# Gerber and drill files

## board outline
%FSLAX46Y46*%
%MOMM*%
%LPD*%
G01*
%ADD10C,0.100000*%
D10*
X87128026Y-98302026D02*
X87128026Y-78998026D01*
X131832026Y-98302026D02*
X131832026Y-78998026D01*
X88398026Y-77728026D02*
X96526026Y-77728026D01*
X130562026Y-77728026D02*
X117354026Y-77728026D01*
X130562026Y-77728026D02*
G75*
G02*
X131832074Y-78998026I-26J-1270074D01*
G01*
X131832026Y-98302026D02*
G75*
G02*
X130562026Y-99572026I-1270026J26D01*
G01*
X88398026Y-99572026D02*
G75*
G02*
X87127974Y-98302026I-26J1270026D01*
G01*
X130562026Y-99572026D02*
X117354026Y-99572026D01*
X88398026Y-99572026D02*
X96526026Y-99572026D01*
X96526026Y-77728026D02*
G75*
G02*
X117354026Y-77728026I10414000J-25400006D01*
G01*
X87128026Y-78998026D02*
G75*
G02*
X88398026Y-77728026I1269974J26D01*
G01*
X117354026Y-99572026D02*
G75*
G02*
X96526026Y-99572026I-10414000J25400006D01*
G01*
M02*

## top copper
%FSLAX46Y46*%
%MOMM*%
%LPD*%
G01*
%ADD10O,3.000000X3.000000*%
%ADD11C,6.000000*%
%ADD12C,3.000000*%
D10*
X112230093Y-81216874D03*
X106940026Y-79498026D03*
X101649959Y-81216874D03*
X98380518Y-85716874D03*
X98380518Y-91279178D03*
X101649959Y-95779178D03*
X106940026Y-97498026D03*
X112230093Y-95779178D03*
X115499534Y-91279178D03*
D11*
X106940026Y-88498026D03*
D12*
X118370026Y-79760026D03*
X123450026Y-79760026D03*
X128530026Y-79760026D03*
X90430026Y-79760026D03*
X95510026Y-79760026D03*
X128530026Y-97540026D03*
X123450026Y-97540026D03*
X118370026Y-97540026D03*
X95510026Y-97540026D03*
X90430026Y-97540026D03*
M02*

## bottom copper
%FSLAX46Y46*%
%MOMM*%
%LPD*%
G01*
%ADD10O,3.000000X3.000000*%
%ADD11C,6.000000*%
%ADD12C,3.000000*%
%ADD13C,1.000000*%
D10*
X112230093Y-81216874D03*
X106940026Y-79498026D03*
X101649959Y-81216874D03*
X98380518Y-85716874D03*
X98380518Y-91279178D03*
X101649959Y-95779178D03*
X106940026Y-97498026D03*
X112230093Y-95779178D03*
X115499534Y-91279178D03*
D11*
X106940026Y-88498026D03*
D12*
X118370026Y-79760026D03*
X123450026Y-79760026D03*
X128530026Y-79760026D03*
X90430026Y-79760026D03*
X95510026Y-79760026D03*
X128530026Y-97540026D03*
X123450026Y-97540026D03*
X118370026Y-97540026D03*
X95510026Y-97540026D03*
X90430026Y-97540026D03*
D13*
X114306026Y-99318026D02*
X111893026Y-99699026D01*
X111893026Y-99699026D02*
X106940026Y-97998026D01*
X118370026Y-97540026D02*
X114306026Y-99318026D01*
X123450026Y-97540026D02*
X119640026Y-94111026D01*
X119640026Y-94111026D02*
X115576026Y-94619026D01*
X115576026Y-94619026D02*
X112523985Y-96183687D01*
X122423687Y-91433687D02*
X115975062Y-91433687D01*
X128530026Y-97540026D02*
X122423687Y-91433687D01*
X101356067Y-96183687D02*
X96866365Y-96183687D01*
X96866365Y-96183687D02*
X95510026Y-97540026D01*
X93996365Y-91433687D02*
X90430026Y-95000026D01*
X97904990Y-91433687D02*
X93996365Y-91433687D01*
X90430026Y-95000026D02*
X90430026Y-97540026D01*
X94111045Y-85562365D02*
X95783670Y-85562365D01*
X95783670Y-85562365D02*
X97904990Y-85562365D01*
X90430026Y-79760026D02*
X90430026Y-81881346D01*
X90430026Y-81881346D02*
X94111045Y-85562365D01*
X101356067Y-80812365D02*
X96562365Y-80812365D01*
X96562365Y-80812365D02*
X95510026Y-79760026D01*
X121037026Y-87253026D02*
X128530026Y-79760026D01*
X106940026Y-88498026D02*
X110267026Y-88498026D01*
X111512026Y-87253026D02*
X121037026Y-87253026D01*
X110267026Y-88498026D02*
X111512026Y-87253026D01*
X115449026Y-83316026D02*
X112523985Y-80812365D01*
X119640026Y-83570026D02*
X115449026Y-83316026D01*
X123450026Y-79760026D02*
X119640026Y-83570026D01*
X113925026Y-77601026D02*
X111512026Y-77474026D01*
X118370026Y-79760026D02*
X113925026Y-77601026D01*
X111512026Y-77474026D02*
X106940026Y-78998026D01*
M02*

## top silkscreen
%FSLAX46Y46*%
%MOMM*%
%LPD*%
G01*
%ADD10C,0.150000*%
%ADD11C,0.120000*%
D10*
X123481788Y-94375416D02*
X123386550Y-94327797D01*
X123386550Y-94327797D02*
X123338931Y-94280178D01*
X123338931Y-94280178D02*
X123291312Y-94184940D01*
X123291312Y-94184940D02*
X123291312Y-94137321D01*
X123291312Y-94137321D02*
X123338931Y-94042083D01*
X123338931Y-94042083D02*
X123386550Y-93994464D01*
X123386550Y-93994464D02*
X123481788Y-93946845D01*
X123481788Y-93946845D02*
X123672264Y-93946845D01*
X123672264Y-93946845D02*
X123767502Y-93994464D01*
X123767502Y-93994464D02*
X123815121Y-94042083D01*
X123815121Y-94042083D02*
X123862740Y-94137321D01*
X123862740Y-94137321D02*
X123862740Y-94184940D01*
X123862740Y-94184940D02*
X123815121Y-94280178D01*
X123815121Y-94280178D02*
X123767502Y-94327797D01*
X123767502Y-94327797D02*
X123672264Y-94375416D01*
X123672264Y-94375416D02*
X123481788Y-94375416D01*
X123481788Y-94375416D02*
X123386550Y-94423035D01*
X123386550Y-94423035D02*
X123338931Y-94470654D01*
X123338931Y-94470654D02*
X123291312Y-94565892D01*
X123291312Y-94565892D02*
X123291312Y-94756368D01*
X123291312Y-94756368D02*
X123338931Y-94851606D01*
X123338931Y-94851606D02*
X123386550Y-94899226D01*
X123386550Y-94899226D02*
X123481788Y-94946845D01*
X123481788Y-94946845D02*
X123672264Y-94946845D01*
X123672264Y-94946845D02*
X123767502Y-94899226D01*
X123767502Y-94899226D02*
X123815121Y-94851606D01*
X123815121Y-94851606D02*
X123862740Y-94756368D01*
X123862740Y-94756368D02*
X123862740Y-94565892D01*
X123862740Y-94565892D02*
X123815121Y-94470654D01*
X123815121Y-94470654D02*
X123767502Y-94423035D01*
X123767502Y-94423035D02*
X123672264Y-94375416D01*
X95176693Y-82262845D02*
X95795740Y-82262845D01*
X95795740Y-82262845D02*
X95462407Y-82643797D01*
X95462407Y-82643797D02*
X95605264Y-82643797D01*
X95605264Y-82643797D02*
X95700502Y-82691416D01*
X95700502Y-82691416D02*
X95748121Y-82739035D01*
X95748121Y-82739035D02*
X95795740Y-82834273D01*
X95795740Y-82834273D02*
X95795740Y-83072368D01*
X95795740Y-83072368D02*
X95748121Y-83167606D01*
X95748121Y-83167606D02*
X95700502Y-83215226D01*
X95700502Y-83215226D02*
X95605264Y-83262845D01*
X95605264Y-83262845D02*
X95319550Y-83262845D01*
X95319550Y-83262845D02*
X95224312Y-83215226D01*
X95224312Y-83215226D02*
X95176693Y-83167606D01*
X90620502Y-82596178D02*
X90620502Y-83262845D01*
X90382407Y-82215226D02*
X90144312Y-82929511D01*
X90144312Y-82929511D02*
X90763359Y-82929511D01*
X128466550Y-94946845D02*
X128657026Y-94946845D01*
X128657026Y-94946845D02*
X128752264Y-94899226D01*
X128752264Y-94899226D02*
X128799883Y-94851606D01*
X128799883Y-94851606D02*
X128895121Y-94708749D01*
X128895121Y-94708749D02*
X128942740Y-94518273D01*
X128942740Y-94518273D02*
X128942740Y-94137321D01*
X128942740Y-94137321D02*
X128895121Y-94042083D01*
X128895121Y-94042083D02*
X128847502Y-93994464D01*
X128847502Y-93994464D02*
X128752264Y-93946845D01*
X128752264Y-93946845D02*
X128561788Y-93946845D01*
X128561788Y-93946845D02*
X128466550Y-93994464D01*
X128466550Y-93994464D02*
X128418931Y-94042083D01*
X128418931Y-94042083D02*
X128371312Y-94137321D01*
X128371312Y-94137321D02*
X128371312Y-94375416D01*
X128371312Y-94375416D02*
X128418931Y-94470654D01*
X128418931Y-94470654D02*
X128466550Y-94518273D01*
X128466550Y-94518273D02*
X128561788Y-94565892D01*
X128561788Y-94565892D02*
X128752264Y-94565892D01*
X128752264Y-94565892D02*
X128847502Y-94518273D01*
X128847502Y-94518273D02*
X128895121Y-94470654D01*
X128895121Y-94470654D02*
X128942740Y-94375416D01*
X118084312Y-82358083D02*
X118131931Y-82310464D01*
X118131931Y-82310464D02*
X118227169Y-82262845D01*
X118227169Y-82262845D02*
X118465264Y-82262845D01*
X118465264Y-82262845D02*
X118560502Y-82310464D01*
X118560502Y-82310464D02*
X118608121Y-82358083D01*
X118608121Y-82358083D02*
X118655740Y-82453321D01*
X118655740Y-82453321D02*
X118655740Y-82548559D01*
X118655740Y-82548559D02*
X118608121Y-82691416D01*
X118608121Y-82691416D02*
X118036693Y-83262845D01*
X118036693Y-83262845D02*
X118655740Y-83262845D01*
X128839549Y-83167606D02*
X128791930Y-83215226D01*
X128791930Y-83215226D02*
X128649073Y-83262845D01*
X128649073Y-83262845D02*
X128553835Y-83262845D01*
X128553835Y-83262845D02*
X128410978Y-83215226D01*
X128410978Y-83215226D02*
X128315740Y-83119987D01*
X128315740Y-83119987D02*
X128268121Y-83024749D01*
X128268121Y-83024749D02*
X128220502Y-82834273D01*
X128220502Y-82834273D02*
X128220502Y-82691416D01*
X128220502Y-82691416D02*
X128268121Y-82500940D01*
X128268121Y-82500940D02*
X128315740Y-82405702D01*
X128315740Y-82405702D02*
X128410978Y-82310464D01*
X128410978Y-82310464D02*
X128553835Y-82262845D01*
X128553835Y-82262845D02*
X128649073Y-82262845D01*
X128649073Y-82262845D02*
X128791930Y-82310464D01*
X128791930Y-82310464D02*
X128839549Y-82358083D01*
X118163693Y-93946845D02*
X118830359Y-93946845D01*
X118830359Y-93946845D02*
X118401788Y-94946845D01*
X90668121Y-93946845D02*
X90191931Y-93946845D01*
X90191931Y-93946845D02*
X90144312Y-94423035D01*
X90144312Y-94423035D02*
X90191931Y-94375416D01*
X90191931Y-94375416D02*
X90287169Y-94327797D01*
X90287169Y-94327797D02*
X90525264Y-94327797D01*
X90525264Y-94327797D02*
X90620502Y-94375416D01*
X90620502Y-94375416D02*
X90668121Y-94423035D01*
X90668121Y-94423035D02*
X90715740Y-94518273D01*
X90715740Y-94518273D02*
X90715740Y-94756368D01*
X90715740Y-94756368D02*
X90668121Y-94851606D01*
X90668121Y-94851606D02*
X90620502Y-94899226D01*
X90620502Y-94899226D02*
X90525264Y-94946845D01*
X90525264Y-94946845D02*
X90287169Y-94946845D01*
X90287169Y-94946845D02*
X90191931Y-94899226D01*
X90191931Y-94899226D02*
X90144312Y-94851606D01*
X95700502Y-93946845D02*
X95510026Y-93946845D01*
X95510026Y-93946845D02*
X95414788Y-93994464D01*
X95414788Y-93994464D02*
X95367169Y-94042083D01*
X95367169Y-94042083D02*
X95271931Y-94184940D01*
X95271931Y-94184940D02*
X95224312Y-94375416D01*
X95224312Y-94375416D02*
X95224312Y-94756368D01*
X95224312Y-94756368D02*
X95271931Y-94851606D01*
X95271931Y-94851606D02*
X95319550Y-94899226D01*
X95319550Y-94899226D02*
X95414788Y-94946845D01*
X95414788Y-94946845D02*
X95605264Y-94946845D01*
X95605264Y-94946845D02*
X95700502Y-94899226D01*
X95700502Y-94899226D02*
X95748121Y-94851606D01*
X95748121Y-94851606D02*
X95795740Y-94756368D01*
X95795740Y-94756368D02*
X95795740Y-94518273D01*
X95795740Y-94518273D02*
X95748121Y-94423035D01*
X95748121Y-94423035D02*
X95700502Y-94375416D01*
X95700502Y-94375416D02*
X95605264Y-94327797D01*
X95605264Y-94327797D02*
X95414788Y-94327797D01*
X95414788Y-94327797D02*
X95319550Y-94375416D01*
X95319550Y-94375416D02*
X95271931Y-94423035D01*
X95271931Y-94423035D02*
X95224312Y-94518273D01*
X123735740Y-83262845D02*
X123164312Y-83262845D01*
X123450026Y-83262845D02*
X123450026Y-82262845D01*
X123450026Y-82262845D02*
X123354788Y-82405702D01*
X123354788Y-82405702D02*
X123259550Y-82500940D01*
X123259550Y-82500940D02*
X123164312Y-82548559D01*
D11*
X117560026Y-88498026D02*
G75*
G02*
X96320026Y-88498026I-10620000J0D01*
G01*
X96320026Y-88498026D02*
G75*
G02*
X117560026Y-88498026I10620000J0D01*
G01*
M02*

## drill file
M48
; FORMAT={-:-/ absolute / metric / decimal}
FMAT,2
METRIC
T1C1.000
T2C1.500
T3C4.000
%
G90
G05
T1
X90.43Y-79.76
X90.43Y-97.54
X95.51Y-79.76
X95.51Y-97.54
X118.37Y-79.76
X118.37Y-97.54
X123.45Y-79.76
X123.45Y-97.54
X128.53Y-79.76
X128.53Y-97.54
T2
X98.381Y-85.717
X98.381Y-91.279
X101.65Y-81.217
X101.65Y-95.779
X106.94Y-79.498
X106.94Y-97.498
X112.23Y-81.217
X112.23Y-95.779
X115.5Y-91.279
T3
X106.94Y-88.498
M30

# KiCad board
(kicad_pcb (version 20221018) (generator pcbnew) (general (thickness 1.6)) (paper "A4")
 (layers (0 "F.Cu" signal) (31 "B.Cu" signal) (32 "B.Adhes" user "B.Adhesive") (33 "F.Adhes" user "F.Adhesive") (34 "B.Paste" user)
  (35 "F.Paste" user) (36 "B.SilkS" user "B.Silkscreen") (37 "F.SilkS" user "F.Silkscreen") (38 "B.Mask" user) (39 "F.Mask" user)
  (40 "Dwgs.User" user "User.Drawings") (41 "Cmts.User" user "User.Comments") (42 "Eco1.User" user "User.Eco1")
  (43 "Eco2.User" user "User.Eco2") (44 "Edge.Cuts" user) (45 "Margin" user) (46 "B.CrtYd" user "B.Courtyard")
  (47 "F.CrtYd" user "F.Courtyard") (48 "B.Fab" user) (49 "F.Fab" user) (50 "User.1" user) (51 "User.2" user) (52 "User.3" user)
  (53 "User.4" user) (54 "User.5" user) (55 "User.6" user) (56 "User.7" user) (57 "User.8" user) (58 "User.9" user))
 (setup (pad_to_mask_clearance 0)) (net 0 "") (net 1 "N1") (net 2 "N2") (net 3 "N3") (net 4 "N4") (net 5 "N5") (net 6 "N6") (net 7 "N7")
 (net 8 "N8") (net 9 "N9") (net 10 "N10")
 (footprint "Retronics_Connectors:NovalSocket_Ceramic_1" (layer "F.Cu") (at 106.940026 88.498026)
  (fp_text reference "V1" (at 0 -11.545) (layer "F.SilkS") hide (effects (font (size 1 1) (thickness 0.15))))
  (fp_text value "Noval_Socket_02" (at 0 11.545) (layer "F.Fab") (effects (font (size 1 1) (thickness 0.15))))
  (fp_circle (center 0 0) (end 0 10.62) (stroke (width 0.12) (type default)) (fill none) (layer "F.SilkS"))
  (pad "1" thru_hole oval (at 5.290067 -7.281152) (size 3 3) (drill 1.5) (layers "*.Cu" "*.Mask") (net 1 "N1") (thermal_bridge_angle 45))
  (pad "2" thru_hole oval (at 0 -9) (size 3 3) (drill 1.5) (layers "*.Cu" "*.Mask") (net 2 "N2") (thermal_bridge_angle 45))
  (pad "3" thru_hole oval (at -5.290067 -7.281152) (size 3 3) (drill 1.5) (layers "*.Cu" "*.Mask") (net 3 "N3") (thermal_bridge_angle 45))
  (pad "4" thru_hole oval (at -8.559508 -2.781152) (size 3 3) (drill 1.5) (layers "*.Cu" "*.Mask") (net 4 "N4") (thermal_bridge_angle 45))
  (pad "5" thru_hole oval (at -8.559508 2.781152) (size 3 3) (drill 1.5) (layers "*.Cu" "*.Mask") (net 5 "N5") (thermal_bridge_angle 45))
  (pad "6" thru_hole oval (at -5.290067 7.281152) (size 3 3) (drill 1.5) (layers "*.Cu" "*.Mask") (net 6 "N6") (thermal_bridge_angle 45))
  (pad "7" thru_hole oval (at 0 9) (size 3 3) (drill 1.5) (layers "*.Cu" "*.Mask") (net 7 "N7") (thermal_bridge_angle 45))
  (pad "8" thru_hole oval (at 5.290067 7.281152) (size 3 3) (drill 1.5) (layers "*.Cu" "*.Mask") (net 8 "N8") (thermal_bridge_angle 45))
  (pad "9" thru_hole oval (at 8.559508 2.781152) (size 3 3) (drill 1.5) (layers "*.Cu" "*.Mask") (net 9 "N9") (thermal_bridge_angle 45))
  (pad "10" thru_hole circle (at 0 0) (size 6 6) (drill 4) (layers "*.Cu" "*.Mask") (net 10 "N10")))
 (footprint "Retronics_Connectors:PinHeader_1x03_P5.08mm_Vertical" (layer "B.Cu") (at 118.370026 79.760026 -90)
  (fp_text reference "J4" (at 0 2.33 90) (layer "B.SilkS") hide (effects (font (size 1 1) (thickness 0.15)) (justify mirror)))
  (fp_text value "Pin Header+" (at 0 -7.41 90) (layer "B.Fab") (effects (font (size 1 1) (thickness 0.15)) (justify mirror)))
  (pad "1" thru_hole circle (at 0 0 270) (size 3 3) (drill 1) (layers "*.Cu" "*.Mask") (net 2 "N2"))
  (pad "2" thru_hole circle (at 0 -5.08 270) (size 3 3) (drill 1) (layers "*.Cu" "*.Mask") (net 1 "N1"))
  (pad "3" thru_hole circle (at 0 -10.16 270) (size 3 3) (drill 1) (layers "*.Cu" "*.Mask") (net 10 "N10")))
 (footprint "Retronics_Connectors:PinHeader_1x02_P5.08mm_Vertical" (layer "B.Cu") (at 90.430026 79.760026 -90)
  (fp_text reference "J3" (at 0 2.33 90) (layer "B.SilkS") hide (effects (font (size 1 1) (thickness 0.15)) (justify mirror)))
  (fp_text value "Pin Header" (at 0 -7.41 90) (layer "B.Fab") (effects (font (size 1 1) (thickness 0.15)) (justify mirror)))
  (pad "1" thru_hole circle (at 0 0 270) (size 3 3) (drill 1) (layers "*.Cu" "*.Mask") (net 4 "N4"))
  (pad "2" thru_hole circle (at 0 -5.08 270) (size 3 3) (drill 1) (layers "*.Cu" "*.Mask") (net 3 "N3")))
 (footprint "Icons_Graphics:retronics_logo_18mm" (layer "B.Cu") (at 121.345721 83.55 180)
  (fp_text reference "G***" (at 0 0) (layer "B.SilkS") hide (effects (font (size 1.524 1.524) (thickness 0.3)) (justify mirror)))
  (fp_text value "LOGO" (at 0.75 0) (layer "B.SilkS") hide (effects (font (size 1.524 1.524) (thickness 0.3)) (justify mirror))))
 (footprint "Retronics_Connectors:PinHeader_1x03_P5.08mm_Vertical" (layer "B.Cu") (at 128.530026 97.540026 90)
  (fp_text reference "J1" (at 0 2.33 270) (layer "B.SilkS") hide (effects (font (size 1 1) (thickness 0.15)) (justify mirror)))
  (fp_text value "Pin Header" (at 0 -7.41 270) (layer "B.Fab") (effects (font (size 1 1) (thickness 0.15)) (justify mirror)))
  (pad "1" thru_hole circle (at 0 0 90) (size 3 3) (drill 1) (layers "*.Cu" "*.Mask") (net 9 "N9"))
  (pad "2" thru_hole circle (at 0 -5.08 90) (size 3 3) (drill 1) (layers "*.Cu" "*.Mask") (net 8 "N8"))
  (pad "3" thru_hole circle (at 0 -10.16 90) (size 3 3) (drill 1) (layers "*.Cu" "*.Mask") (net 7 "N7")))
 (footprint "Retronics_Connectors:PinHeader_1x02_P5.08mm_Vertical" (layer "B.Cu") (at 95.510026 97.540026 90)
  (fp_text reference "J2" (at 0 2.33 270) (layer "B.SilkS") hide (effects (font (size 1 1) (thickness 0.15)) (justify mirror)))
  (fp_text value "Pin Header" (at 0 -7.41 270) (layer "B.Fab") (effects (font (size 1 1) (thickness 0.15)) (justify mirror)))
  (pad "1" thru_hole circle (at 0 0 90) (size 3 3) (drill 1) (layers "*.Cu" "*.Mask") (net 6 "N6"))
  (pad "2" thru_hole circle (at 0 -5.08 90) (size 3 3) (drill 1) (layers "*.Cu" "*.Mask") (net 5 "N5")))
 (gr_line (start 87.128026 98.302026) (end 87.128026 78.998026) (stroke (width 0.1) (type solid)) (layer "Edge.Cuts"))
 (gr_line (start 131.832026 98.302026) (end 131.832026 78.998026) (stroke (width 0.1) (type solid)) (layer "Edge.Cuts"))
 (gr_line (start 88.398026 77.728026) (end 96.526026 77.728026) (stroke (width 0.1) (type solid)) (layer "Edge.Cuts"))
 (gr_line (start 130.562026 77.728026) (end 117.354026 77.728026) (stroke (width 0.1) (type solid)) (layer "Edge.Cuts"))
 (gr_arc (start 130.562026 77.728026) (mid 131.460026 78.100011) (end 131.832026 78.998026) (stroke (width 0.1) (type solid))
  (layer "Edge.Cuts"))
 (gr_arc (start 131.832026 98.302026) (mid 131.460044 99.200044) (end 130.562026 99.572026) (stroke (width 0.1) (type solid))
  (layer "Edge.Cuts"))
 (gr_arc (start 88.398026 99.572026) (mid 87.5 99.200052) (end 87.128026 98.302026) (stroke (width 0.1) (type solid)) (layer "Edge.Cuts"))
 (gr_line (start 130.562026 99.572026) (end 117.354026 99.572026) (stroke (width 0.1) (type solid)) (layer "Edge.Cuts"))
 (gr_line (start 88.398026 99.572026) (end 96.526026 99.572026) (stroke (width 0.1) (type solid)) (layer "Edge.Cuts"))
 (gr_arc (start 96.526026 77.728026) (mid 106.940026 75.676043) (end 117.354026 77.728026) (stroke (width 0.1) (type solid))
  (layer "Edge.Cuts"))
 (gr_arc (start 87.128026 78.998026) (mid 87.5 78.1) (end 88.398026 77.728026) (stroke (width 0.1) (type solid)) (layer "Edge.Cuts"))
 (gr_arc (start 117.354026 99.572026) (mid 106.940026 101.624009) (end 96.526026 99.572026) (stroke (width 0.1) (type solid))
  (layer "Edge.Cuts"))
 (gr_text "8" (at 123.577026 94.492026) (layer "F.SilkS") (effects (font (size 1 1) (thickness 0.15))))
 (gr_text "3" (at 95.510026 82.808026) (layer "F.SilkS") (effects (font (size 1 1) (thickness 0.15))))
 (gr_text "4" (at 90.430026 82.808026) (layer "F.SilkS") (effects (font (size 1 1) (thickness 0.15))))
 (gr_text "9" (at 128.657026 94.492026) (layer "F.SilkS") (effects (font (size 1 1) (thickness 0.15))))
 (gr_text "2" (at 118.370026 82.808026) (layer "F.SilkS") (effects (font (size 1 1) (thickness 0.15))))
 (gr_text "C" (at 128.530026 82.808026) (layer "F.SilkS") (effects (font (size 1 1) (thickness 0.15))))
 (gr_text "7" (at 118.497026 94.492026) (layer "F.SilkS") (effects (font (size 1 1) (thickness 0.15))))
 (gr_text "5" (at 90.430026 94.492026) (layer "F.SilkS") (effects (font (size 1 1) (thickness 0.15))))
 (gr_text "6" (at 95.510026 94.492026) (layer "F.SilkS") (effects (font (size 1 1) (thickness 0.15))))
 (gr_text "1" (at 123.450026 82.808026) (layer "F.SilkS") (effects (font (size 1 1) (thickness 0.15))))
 (segment (start 114.306026 99.318026) (end 111.893026 99.699026) (width 1) (layer "B.Cu") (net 7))
 (segment (start 111.893026 99.699026) (end 106.940026 97.998026) (width 1) (layer "B.Cu") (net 7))
 (segment (start 118.370026 97.540026) (end 114.306026 99.318026) (width 1) (layer "B.Cu") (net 7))
 (segment (start 123.450026 97.540026) (end 119.640026 94.111026) (width 1) (layer "B.Cu") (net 8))
 (segment (start 119.640026 94.111026) (end 115.576026 94.619026) (width 1) (layer "B.Cu") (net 8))
 (segment (start 115.576026 94.619026) (end 112.523985 96.183687) (width 1) (layer "B.Cu") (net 8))
 (segment (start 122.423687 91.433687) (end 115.975062 91.433687) (width 1) (layer "B.Cu") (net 9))
 (segment (start 128.530026 97.540026) (end 122.423687 91.433687) (width 1) (layer "B.Cu") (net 9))
 (segment (start 101.356067 96.183687) (end 96.866365 96.183687) (width 1) (layer "B.Cu") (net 6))
 (segment (start 96.866365 96.183687) (end 95.510026 97.540026) (width 1) (layer "B.Cu") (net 6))
 (segment (start 93.996365 91.433687) (end 90.430026 95.000026) (width 1) (layer "B.Cu") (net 5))
 (segment (start 97.90499 91.433687) (end 93.996365 91.433687) (width 1) (layer "B.Cu") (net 5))
 (segment (start 90.430026 95.000026) (end 90.430026 97.540026) (width 1) (layer "B.Cu") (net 5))
 (segment (start 94.111045 85.562365) (end 95.78367 85.562365) (width 1) (layer "B.Cu") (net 4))
 (segment (start 95.78367 85.562365) (end 97.90499 85.562365) (width 1) (layer "B.Cu") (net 4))
 (segment (start 90.430026 79.760026) (end 90.430026 81.881346) (width 1) (layer "B.Cu") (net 4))
 (segment (start 90.430026 81.881346) (end 94.111045 85.562365) (width 1) (layer "B.Cu") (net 4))
 (segment (start 101.356067 80.812365) (end 96.562365 80.812365) (width 1) (layer "B.Cu") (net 3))
 (segment (start 96.562365 80.812365) (end 95.510026 79.760026) (width 1) (layer "B.Cu") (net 3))
 (segment (start 121.037026 87.253026) (end 128.530026 79.760026) (width 1) (layer "B.Cu") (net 10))
 (segment (start 106.940026 88.498026) (end 110.267026 88.498026) (width 1) (layer "B.Cu") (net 10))
 (segment (start 111.512026 87.253026) (end 121.037026 87.253026) (width 1) (layer "B.Cu") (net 10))
 (segment (start 110.267026 88.498026) (end 111.512026 87.253026) (width 1) (layer "B.Cu") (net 10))
 (segment (start 115.449026 83.316026) (end 112.523985 80.812365) (width 1) (layer "B.Cu") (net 1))
 (segment (start 119.640026 83.570026) (end 115.449026 83.316026) (width 1) (layer "B.Cu") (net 1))
 (segment (start 123.450026 79.760026) (end 119.640026 83.570026) (width 1) (layer "B.Cu") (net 1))
 (segment (start 113.925026 77.601026) (end 111.512026 77.474026) (width 1) (layer "B.Cu") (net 2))
 (segment (start 118.370026 79.760026) (end 113.925026 77.601026) (width 1) (layer "B.Cu") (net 2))
 (segment (start 111.512026 77.474026) (end 106.940026 78.998026) (width 1) (layer "B.Cu") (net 2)))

